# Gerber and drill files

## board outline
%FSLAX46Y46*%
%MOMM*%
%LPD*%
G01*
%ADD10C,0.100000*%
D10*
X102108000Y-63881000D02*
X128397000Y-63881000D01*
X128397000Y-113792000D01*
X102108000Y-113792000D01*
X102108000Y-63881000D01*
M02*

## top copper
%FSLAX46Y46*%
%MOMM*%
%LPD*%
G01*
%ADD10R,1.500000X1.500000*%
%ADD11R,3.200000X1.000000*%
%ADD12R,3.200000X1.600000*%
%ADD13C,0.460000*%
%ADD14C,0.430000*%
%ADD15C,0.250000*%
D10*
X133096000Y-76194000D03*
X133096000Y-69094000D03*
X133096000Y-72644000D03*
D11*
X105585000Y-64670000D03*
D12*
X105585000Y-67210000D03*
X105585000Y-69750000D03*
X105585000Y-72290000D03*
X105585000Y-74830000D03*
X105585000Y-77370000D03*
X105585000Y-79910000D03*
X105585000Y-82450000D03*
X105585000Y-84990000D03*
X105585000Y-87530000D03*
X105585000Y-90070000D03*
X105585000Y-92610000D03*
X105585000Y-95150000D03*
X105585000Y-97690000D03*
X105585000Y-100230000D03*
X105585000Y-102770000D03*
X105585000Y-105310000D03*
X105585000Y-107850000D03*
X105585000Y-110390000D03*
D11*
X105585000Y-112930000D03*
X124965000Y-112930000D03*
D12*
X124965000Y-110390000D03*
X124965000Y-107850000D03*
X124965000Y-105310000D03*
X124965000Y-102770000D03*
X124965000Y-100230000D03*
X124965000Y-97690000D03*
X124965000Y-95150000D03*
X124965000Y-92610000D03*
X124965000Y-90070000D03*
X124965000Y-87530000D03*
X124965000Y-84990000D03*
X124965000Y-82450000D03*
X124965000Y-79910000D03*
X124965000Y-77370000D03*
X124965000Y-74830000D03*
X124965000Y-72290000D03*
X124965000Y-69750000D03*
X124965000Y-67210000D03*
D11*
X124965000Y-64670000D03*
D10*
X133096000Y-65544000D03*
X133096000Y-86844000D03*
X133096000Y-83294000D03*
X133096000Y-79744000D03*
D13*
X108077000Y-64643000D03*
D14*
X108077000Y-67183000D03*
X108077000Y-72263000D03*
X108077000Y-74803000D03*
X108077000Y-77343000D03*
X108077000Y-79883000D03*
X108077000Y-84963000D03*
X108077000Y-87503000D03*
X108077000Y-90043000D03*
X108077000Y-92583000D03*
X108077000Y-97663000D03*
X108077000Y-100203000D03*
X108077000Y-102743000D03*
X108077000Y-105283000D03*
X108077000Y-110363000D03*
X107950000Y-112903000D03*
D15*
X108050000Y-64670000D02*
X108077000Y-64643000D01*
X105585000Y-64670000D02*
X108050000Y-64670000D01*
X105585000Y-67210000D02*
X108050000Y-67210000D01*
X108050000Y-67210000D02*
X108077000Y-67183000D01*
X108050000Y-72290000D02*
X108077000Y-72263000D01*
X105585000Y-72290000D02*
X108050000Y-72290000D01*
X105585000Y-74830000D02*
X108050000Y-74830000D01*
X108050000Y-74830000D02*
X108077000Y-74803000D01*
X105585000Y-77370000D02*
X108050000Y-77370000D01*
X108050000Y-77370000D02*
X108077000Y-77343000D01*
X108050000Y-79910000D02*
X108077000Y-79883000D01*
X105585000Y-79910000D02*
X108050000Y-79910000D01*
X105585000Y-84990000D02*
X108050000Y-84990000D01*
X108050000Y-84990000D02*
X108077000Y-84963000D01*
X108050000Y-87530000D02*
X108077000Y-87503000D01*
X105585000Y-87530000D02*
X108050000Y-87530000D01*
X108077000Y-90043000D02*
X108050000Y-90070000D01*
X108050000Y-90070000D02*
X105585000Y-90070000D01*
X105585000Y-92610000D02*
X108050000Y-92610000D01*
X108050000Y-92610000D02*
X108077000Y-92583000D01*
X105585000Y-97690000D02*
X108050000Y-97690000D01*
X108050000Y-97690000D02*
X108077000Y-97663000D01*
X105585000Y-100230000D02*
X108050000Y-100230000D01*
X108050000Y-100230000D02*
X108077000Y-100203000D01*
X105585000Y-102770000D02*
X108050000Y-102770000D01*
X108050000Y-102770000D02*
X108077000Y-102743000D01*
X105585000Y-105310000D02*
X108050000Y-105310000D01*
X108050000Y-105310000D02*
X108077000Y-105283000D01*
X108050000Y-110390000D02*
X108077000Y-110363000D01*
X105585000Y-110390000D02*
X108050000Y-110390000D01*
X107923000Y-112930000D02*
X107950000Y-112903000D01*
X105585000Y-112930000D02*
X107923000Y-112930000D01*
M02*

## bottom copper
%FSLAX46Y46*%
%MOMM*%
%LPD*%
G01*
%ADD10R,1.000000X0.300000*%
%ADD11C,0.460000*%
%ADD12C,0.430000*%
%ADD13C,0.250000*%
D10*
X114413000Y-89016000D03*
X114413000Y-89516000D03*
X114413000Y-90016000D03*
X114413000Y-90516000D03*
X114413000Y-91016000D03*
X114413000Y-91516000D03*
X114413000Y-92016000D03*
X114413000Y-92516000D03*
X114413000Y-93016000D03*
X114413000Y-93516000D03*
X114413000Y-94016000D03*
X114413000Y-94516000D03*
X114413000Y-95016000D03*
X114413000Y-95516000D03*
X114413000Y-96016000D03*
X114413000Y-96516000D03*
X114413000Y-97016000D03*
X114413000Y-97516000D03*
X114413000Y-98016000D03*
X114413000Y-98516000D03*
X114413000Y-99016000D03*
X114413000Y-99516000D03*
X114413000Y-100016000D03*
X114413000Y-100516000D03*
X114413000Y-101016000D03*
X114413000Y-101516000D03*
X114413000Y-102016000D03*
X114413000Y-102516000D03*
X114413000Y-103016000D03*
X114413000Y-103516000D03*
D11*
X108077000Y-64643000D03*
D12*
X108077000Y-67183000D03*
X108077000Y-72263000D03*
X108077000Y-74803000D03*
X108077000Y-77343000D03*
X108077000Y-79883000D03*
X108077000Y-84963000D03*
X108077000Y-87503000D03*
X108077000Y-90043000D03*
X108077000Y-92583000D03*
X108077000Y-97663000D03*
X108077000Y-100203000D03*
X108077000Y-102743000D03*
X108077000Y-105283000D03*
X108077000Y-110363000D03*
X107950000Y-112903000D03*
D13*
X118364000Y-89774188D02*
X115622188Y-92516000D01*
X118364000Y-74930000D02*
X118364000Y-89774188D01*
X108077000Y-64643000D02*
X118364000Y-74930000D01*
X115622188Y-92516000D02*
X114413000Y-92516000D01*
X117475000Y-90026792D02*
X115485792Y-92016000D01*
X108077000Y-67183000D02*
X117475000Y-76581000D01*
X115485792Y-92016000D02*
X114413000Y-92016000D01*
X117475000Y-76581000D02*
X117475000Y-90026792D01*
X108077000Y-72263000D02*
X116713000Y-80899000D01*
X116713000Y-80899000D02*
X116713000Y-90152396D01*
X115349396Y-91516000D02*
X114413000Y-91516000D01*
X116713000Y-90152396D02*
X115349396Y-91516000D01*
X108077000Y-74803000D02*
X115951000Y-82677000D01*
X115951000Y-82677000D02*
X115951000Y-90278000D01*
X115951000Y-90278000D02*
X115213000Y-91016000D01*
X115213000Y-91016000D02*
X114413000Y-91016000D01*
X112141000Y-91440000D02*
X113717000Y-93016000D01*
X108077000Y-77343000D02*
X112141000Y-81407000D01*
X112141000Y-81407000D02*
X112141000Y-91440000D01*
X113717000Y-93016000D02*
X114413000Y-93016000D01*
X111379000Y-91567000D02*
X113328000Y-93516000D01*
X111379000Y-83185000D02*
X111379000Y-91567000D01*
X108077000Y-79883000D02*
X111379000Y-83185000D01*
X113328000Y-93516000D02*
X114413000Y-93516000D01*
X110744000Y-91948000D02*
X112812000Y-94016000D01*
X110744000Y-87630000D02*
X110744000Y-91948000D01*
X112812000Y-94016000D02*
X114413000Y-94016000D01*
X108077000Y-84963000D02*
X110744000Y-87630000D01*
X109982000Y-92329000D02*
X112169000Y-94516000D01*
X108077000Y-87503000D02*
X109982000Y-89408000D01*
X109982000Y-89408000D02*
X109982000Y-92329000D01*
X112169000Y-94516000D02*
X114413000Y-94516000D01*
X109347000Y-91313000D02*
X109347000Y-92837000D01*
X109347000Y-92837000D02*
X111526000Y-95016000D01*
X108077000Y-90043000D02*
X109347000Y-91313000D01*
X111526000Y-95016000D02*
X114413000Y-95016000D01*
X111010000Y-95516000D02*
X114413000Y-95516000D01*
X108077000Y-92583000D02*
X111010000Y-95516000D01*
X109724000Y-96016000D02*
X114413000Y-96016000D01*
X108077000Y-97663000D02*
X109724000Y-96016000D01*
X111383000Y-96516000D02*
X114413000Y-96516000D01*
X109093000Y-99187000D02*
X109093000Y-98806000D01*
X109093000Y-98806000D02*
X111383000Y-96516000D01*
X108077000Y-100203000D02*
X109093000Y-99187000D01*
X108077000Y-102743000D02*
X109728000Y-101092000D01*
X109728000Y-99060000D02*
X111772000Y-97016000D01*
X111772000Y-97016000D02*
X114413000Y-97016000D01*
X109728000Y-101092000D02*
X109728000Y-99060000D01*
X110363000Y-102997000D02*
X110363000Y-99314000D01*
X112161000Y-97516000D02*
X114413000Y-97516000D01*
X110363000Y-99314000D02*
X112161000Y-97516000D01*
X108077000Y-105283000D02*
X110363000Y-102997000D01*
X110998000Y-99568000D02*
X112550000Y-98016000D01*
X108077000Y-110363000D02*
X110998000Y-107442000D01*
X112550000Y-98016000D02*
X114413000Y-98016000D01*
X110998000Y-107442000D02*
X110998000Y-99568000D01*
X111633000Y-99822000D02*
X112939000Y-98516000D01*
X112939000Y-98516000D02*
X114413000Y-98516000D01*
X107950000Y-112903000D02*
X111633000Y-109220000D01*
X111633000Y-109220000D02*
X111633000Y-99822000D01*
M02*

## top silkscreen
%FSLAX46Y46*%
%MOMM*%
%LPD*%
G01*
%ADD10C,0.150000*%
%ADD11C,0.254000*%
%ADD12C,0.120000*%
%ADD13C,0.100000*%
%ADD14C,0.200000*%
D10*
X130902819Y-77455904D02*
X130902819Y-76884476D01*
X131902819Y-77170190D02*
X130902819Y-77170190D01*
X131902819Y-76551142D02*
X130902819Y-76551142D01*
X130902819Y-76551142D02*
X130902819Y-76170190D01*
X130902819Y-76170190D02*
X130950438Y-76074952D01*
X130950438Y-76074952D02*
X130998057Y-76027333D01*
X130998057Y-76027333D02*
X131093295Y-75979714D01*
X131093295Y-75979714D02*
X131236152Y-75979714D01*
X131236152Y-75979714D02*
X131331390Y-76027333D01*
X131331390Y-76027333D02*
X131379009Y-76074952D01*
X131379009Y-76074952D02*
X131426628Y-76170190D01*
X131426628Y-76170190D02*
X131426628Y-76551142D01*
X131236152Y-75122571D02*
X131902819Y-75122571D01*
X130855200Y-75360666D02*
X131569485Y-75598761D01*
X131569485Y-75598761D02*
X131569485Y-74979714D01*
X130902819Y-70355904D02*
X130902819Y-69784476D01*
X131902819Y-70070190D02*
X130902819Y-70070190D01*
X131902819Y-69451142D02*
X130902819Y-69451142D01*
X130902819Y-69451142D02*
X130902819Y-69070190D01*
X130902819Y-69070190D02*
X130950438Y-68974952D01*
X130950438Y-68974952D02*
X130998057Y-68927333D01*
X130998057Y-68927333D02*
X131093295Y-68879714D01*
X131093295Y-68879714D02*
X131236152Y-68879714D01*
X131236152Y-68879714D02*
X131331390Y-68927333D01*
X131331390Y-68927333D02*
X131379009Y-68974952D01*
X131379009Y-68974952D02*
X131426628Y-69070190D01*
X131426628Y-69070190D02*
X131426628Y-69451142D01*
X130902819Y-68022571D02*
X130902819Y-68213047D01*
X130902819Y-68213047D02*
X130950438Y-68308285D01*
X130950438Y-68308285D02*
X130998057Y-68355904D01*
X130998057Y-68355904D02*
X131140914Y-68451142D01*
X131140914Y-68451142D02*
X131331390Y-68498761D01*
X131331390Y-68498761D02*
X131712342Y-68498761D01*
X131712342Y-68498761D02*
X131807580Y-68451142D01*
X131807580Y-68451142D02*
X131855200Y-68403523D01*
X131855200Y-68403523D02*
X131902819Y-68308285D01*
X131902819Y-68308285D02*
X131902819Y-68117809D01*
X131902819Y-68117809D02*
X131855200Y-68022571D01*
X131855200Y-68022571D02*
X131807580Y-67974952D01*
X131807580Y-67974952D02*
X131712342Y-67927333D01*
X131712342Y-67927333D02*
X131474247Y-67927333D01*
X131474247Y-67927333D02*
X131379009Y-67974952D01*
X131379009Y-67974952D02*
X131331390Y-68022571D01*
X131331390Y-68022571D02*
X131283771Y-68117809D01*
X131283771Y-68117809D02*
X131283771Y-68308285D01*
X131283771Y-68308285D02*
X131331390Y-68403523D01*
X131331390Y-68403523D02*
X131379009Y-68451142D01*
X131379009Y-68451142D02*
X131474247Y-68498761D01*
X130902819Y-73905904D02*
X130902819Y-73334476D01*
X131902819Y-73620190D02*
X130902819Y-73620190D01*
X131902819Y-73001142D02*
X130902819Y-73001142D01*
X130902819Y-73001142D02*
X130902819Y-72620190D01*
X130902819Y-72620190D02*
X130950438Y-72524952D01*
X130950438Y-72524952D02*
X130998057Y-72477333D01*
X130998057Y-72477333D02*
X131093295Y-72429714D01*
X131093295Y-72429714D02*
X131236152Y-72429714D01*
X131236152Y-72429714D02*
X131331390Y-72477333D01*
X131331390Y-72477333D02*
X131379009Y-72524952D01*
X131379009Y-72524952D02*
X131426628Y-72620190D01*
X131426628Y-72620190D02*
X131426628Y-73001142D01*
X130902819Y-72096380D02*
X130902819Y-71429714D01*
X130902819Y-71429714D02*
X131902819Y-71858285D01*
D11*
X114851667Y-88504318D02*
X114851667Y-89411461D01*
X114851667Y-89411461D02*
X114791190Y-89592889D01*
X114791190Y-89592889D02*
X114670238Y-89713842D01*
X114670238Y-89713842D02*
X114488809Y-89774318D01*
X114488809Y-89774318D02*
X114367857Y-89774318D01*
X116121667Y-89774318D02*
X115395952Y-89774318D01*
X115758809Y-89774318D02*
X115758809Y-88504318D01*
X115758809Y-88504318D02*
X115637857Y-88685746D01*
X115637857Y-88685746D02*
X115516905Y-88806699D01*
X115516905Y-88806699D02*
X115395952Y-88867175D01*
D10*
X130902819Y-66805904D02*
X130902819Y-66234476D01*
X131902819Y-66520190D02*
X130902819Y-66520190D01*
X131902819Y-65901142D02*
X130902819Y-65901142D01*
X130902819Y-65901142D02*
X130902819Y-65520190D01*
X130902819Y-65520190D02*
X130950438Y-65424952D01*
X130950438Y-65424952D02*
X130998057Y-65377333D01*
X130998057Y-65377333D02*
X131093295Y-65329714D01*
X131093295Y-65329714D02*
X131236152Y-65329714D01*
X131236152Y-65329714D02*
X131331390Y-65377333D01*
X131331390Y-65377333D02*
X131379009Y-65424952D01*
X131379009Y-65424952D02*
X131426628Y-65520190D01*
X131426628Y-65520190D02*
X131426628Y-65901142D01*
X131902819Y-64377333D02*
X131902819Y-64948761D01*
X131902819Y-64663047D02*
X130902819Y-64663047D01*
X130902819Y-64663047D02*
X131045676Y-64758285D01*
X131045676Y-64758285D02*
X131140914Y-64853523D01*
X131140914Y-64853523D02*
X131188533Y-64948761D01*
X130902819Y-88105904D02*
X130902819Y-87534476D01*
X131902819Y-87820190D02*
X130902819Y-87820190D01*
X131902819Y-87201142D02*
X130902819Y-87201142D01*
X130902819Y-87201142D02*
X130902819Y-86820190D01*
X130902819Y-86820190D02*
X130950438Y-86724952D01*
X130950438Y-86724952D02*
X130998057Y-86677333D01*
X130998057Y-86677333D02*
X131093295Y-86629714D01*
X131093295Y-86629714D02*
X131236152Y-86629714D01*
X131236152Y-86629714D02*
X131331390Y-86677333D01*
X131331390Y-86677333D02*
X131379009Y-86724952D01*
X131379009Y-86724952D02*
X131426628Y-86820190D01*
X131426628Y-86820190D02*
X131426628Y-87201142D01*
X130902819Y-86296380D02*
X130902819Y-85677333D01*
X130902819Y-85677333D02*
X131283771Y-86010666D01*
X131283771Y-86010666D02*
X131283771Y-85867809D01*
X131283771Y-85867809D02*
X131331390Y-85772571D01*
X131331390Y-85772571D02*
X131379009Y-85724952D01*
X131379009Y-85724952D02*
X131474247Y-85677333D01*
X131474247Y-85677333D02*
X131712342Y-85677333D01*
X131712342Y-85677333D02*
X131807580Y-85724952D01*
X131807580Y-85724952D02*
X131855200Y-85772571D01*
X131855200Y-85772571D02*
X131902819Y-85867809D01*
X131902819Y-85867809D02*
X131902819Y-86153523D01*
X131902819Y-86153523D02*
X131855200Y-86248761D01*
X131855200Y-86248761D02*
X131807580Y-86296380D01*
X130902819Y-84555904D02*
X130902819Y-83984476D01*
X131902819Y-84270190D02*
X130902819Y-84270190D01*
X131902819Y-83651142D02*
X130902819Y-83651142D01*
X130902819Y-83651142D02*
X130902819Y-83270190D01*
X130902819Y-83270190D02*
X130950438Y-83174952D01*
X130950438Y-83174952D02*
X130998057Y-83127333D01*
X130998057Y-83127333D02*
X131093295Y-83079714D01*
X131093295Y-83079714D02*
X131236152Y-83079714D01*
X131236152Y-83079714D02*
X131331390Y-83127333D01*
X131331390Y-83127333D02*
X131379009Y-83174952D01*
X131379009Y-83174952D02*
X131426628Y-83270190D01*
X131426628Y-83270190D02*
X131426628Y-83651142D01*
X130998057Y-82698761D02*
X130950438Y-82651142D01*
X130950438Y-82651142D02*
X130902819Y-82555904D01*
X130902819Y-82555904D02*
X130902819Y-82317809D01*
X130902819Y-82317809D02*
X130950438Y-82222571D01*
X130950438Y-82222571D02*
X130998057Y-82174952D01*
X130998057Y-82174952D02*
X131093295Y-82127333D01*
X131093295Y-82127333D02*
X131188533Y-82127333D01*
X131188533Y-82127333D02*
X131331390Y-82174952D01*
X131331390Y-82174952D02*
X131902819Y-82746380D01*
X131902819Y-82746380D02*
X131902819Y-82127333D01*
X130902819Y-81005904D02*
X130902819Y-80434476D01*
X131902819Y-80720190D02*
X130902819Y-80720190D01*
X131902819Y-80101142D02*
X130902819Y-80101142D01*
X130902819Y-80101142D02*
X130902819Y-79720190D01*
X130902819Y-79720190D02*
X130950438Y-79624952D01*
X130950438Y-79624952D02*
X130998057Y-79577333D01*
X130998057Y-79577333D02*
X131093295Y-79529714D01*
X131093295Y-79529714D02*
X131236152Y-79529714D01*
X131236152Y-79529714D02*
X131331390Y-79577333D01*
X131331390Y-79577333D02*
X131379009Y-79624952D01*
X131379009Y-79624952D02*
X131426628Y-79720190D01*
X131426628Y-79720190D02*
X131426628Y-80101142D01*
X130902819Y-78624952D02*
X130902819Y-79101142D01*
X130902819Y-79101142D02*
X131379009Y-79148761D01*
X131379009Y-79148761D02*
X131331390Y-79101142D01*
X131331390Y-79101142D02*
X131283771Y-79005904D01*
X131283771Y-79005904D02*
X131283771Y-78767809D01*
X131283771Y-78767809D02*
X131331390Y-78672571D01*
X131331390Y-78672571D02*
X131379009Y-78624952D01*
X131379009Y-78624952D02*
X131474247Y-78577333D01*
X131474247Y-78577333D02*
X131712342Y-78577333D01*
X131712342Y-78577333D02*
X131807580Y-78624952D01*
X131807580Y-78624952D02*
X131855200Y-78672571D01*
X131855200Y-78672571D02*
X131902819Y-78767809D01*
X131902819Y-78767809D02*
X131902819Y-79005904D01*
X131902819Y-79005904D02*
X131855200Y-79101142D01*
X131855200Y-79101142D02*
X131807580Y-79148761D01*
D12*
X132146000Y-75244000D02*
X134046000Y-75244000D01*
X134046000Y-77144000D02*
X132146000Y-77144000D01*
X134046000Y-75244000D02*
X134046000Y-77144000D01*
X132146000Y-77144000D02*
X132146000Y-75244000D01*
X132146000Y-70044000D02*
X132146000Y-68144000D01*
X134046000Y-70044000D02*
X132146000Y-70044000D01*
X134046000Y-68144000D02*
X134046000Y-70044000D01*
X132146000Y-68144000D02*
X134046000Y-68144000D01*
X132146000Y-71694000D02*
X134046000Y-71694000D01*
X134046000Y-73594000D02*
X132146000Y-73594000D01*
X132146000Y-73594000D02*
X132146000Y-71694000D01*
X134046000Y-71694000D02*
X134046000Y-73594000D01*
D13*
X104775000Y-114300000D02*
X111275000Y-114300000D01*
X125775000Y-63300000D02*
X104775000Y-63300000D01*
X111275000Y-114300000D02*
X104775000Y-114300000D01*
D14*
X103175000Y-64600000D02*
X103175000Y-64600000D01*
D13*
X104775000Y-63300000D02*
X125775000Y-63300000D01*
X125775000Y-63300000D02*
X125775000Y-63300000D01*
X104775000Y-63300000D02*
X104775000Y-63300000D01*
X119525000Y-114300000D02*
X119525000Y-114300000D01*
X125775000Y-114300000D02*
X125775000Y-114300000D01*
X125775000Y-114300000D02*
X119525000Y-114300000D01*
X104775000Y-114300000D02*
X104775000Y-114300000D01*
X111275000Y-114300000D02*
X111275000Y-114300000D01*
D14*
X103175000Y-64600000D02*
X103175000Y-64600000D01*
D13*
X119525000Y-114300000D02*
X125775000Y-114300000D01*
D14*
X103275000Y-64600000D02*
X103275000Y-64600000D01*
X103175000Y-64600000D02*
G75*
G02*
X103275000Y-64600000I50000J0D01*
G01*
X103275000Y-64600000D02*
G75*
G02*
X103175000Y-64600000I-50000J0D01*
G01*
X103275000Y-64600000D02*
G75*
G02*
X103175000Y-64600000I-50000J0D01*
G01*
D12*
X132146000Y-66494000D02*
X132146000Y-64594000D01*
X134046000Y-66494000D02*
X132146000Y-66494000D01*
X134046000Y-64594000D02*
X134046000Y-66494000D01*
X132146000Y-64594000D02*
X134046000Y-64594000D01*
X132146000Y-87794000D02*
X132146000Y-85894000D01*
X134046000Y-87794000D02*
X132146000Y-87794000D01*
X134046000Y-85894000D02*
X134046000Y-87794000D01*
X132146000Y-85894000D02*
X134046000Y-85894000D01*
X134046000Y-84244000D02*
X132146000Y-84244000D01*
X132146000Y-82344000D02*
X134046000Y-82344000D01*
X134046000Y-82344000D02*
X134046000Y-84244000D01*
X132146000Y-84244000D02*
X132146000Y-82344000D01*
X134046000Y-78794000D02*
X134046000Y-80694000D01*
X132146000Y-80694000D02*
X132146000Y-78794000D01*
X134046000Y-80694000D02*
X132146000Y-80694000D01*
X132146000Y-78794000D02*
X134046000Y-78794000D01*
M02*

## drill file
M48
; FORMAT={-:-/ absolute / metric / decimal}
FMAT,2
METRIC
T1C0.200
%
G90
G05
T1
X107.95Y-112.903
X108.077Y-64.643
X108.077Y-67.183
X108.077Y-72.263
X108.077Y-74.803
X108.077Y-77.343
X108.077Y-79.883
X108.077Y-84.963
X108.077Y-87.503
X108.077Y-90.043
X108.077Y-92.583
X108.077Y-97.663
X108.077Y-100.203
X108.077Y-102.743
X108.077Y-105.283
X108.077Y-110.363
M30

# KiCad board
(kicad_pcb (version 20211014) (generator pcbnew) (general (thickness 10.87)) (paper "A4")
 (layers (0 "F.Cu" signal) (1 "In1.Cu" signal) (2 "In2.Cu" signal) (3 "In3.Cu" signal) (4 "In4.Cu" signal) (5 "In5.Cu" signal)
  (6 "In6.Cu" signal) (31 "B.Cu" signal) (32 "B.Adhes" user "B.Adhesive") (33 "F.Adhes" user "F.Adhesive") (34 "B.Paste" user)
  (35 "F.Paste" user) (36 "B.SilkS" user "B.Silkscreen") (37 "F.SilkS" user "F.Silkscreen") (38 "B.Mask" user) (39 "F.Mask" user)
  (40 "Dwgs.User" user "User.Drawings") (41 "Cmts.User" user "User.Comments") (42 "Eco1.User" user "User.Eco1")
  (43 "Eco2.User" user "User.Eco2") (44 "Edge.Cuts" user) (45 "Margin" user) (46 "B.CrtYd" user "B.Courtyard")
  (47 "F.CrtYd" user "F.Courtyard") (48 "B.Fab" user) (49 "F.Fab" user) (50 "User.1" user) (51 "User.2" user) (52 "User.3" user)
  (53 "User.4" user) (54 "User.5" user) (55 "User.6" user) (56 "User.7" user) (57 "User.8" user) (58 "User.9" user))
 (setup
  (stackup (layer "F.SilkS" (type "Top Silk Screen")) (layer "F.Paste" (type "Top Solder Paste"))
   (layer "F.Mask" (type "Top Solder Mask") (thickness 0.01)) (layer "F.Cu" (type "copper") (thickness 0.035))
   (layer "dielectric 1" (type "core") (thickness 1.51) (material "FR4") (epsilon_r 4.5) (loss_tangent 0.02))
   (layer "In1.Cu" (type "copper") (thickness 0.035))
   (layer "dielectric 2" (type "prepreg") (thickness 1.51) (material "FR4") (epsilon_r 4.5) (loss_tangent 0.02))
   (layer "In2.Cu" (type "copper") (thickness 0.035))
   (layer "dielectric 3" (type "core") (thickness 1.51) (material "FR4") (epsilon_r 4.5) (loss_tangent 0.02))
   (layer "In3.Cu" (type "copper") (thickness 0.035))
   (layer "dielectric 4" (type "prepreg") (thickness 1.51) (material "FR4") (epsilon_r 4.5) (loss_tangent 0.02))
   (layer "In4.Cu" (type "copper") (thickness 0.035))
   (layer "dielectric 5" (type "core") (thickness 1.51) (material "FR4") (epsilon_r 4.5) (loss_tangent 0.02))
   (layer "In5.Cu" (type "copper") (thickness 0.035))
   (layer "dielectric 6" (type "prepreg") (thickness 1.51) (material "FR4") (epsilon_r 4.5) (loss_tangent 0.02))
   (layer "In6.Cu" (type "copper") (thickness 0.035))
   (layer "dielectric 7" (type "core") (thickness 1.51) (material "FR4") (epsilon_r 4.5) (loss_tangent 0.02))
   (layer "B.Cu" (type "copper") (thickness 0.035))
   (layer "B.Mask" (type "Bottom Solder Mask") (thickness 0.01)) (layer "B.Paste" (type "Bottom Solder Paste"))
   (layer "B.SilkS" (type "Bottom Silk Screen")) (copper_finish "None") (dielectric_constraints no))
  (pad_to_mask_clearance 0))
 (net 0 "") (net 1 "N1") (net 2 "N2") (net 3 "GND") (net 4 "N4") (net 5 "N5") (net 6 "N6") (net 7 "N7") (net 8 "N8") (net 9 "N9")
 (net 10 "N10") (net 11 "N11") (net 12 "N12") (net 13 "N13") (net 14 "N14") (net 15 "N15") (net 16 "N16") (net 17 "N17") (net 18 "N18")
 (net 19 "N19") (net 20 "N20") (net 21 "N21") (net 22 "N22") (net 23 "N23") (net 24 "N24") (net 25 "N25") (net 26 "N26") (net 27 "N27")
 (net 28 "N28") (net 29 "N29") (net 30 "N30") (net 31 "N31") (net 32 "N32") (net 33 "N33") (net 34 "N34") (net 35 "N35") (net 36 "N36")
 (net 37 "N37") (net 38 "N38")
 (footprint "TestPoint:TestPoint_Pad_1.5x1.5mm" (layer "F.Cu") (at 133.096 76.194 90)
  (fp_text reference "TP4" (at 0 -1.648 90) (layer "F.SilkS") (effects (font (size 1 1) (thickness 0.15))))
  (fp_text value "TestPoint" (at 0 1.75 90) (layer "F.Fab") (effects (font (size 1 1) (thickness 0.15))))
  (fp_line (start 0.95 -0.95) (end 0.95 0.95) (layer "F.SilkS") (width 0.12))
  (fp_line (start -0.95 0.95) (end -0.95 -0.95) (layer "F.SilkS") (width 0.12))
  (fp_line (start 0.95 0.95) (end -0.95 0.95) (layer "F.SilkS") (width 0.12))
  (fp_line (start -0.95 -0.95) (end 0.95 -0.95) (layer "F.SilkS") (width 0.12))
  (pad "1" smd rect (at 0 0 90) (size 1.5 1.5) (layers "F.Cu" "F.Mask") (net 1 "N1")))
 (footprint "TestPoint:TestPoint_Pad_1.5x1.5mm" (layer "F.Cu") (at 133.096 69.094 90)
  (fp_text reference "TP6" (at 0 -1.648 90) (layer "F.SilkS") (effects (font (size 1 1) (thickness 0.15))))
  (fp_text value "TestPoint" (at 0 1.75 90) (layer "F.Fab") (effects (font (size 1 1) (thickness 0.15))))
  (fp_line (start -0.95 -0.95) (end 0.95 -0.95) (layer "F.SilkS") (width 0.12))
  (fp_line (start -0.95 0.95) (end -0.95 -0.95) (layer "F.SilkS") (width 0.12))
  (fp_line (start 0.95 0.95) (end -0.95 0.95) (layer "F.SilkS") (width 0.12))
  (fp_line (start 0.95 -0.95) (end 0.95 0.95) (layer "F.SilkS") (width 0.12))
  (pad "1" smd rect (at 0 0 90) (size 1.5 1.5) (layers "F.Cu" "F.Mask") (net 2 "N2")))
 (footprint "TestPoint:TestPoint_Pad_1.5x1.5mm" (layer "F.Cu") (at 133.096 72.644 90)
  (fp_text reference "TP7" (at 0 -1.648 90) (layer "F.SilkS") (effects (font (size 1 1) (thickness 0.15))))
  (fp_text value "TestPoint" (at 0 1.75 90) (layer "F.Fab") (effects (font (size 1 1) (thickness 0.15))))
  (fp_line (start 0.95 -0.95) (end 0.95 0.95) (layer "F.SilkS") (width 0.12))
  (fp_line (start -0.95 0.95) (end -0.95 -0.95) (layer "F.SilkS") (width 0.12))
  (fp_line (start -0.95 -0.95) (end 0.95 -0.95) (layer "F.SilkS") (width 0.12))
  (fp_line (start 0.95 0.95) (end -0.95 0.95) (layer "F.SilkS") (width 0.12))
  (pad "1" smd rect (at 0 0 90) (size 1.5 1.5) (layers "F.Cu" "F.Mask") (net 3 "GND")))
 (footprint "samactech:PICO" (layer "F.Cu") (at 104.775 114.3)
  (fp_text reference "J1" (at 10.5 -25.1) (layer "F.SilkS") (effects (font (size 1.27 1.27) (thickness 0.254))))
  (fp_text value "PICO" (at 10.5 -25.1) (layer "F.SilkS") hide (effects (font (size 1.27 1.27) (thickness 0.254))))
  (fp_line (start 0 0) (end 6.5 0) (layer "F.SilkS") (width 0.1))
  (fp_line (start 21 -51) (end 0 -51) (layer "F.SilkS") (width 0.1))
  (fp_line (start 6.5 0) (end 0 0) (layer "F.SilkS") (width 0.1))
  (fp_line (start -1.6 -49.7) (end -1.6 -49.7) (layer "F.SilkS") (width 0.2))
  (fp_line (start 0 -51) (end 21 -51) (layer "F.SilkS") (width 0.1))
  (fp_line (start 21 -51) (end 21 -51) (layer "F.SilkS") (width 0.1))
  (fp_line (start 0 -51) (end 0 -51) (layer "F.SilkS") (width 0.1))
  (fp_line (start 14.75 0) (end 14.75 0) (layer "F.SilkS") (width 0.1))
  (fp_line (start 21 0) (end 21 0) (layer "F.SilkS") (width 0.1))
  (fp_line (start 21 0) (end 14.75 0) (layer "F.SilkS") (width 0.1))
  (fp_line (start 0 0) (end 0 0) (layer "F.SilkS") (width 0.1))
  (fp_line (start 6.5 0) (end 6.5 0) (layer "F.SilkS") (width 0.1))
  (fp_line (start -1.6 -49.7) (end -1.6 -49.7) (layer "F.SilkS") (width 0.2))
  (fp_line (start 14.75 0) (end 21 0) (layer "F.SilkS") (width 0.1))
  (fp_line (start -1.5 -49.7) (end -1.5 -49.7) (layer "F.SilkS") (width 0.2))
  (fp_arc (start -1.6 -49.7) (mid -1.55 -49.75) (end -1.5 -49.7) (layer "F.SilkS") (width 0.2))
  (fp_arc (start -1.5 -49.7) (mid -1.55 -49.65) (end -1.6 -49.7) (layer "F.SilkS") (width 0.2))
  (fp_arc (start -1.5 -49.7) (mid -1.55 -49.65) (end -1.6 -49.7) (layer "F.SilkS") (width 0.2))
  (pad "1" smd rect (at 0.81 -49.63 90) (size 1 3.2) (layers "F.Cu" "F.Paste" "F.Mask") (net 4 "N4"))
  (pad "2" smd rect (at 0.81 -47.09 90) (size 1.6 3.2) (layers "F.Cu" "F.Paste" "F.Mask") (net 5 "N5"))
  (pad "3" smd rect (at 0.81 -44.55 90) (size 1.6 3.2) (layers "F.Cu" "F.Paste" "F.Mask") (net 3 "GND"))
  (pad "4" smd rect (at 0.81 -42.01 90) (size 1.6 3.2) (layers "F.Cu" "F.Paste" "F.Mask") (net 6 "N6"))
  (pad "5" smd rect (at 0.81 -39.47 90) (size 1.6 3.2) (layers "F.Cu" "F.Paste" "F.Mask") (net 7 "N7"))
  (pad "6" smd rect (at 0.81 -36.93 90) (size 1.6 3.2) (layers "F.Cu" "F.Paste" "F.Mask") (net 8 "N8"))
  (pad "7" smd rect (at 0.81 -34.39 90) (size 1.6 3.2) (layers "F.Cu" "F.Paste" "F.Mask") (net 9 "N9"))
  (pad "8" smd rect (at 0.81 -31.85 90) (size 1.6 3.2) (layers "F.Cu" "F.Paste" "F.Mask") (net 3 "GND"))
  (pad "9" smd rect (at 0.81 -29.31 90) (size 1.6 3.2) (layers "F.Cu" "F.Paste" "F.Mask") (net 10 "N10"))
  (pad "10" smd rect (at 0.81 -26.77 90) (size 1.6 3.2) (layers "F.Cu" "F.Paste" "F.Mask") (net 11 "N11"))
  (pad "11" smd rect (at 0.81 -24.23 90) (size 1.6 3.2) (layers "F.Cu" "F.Paste" "F.Mask") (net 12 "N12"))
  (pad "12" smd rect (at 0.81 -21.69 90) (size 1.6 3.2) (layers "F.Cu" "F.Paste" "F.Mask") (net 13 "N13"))
  (pad "13" smd rect (at 0.81 -19.15 90) (size 1.6 3.2) (layers "F.Cu" "F.Paste" "F.Mask") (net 3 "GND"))
  (pad "14" smd rect (at 0.81 -16.61 90) (size 1.6 3.2) (layers "F.Cu" "F.Paste" "F.Mask") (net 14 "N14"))
  (pad "15" smd rect (at 0.81 -14.07 90) (size 1.6 3.2) (layers "F.Cu" "F.Paste" "F.Mask") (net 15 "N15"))
  (pad "16" smd rect (at 0.81 -11.53 90) (size 1.6 3.2) (layers "F.Cu" "F.Paste" "F.Mask") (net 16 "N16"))
  (pad "17" smd rect (at 0.81 -8.99 90) (size 1.6 3.2) (layers "F.Cu" "F.Paste" "F.Mask") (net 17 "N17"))
  (pad "18" smd rect (at 0.81 -6.45 90) (size 1.6 3.2) (layers "F.Cu" "F.Paste" "F.Mask") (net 3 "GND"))
  (pad "19" smd rect (at 0.81 -3.91 90) (size 1.6 3.2) (layers "F.Cu" "F.Paste" "F.Mask") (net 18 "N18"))
  (pad "20" smd rect (at 0.81 -1.37 90) (size 1 3.2) (layers "F.Cu" "F.Paste" "F.Mask") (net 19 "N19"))
  (pad "21" smd rect (at 20.19 -1.37 90) (size 1 3.2) (layers "F.Cu" "F.Paste" "F.Mask") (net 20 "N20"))
  (pad "22" smd rect (at 20.19 -3.91 90) (size 1.6 3.2) (layers "F.Cu" "F.Paste" "F.Mask") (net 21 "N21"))
  (pad "23" smd rect (at 20.19 -6.45 90) (size 1.6 3.2) (layers "F.Cu" "F.Paste" "F.Mask") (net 3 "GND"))
  (pad "24" smd rect (at 20.19 -8.99 90) (size 1.6 3.2) (layers "F.Cu" "F.Paste" "F.Mask") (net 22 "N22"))
  (pad "25" smd rect (at 20.19 -11.53 90) (size 1.6 3.2) (layers "F.Cu" "F.Paste" "F.Mask") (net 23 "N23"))
  (pad "26" smd rect (at 20.19 -14.07 90) (size 1.6 3.2) (layers "F.Cu" "F.Paste" "F.Mask") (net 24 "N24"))
  (pad "27" smd rect (at 20.19 -16.61 90) (size 1.6 3.2) (layers "F.Cu" "F.Paste" "F.Mask") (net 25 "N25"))
  (pad "28" smd rect (at 20.19 -19.15 90) (size 1.6 3.2) (layers "F.Cu" "F.Paste" "F.Mask") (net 3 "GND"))
  (pad "29" smd rect (at 20.19 -21.69 90) (size 1.6 3.2) (layers "F.Cu" "F.Paste" "F.Mask") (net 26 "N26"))
  (pad "30" smd rect (at 20.19 -24.23 90) (size 1.6 3.2) (layers "F.Cu" "F.Paste" "F.Mask") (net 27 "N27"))
  (pad "31" smd rect (at 20.19 -26.77 90) (size 1.6 3.2) (layers "F.Cu" "F.Paste" "F.Mask") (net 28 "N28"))
  (pad "32" smd rect (at 20.19 -29.31 90) (size 1.6 3.2) (layers "F.Cu" "F.Paste" "F.Mask") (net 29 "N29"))
  (pad "33" smd rect (at 20.19 -31.85 90) (size 1.6 3.2) (layers "F.Cu" "F.Paste" "F.Mask") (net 3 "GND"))
  (pad "34" smd rect (at 20.19 -34.39 90) (size 1.6 3.2) (layers "F.Cu" "F.Paste" "F.Mask") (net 2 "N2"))
  (pad "35" smd rect (at 20.19 -36.93 90) (size 1.6 3.2) (layers "F.Cu" "F.Paste" "F.Mask") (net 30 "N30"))
  (pad "36" smd rect (at 20.19 -39.47 90) (size 1.6 3.2) (layers "F.Cu" "F.Paste" "F.Mask") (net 1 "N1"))
  (pad "37" smd rect (at 20.19 -42.01 90) (size 1.6 3.2) (layers "F.Cu" "F.Paste" "F.Mask") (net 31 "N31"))
  (pad "38" smd rect (at 20.19 -44.55 90) (size 1.6 3.2) (layers "F.Cu" "F.Paste" "F.Mask") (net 3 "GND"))
  (pad "39" smd rect (at 20.19 -47.09 90) (size 1.6 3.2) (layers "F.Cu" "F.Paste" "F.Mask") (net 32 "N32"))
  (pad "40" smd rect (at 20.19 -49.63 90) (size 1 3.2) (layers "F.Cu" "F.Paste" "F.Mask") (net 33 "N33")))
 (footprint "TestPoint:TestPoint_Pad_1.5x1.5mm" (layer "F.Cu") (at 133.096 65.544 90)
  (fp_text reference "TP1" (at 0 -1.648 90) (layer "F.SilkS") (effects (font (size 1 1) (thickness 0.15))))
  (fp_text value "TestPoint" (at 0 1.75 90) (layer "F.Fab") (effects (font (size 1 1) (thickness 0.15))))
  (fp_line (start -0.95 -0.95) (end 0.95 -0.95) (layer "F.SilkS") (width 0.12))
  (fp_line (start -0.95 0.95) (end -0.95 -0.95) (layer "F.SilkS") (width 0.12))
  (fp_line (start 0.95 0.95) (end -0.95 0.95) (layer "F.SilkS") (width 0.12))
  (fp_line (start 0.95 -0.95) (end 0.95 0.95) (layer "F.SilkS") (width 0.12))
  (pad "1" smd rect (at 0 0 90) (size 1.5 1.5) (layers "F.Cu" "F.Mask") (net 33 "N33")))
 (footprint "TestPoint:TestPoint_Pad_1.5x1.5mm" (layer "F.Cu") (at 133.096 86.844 90)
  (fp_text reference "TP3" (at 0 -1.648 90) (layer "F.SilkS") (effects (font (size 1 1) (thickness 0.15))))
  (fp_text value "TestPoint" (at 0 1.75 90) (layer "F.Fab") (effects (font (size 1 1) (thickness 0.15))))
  (fp_line (start -0.95 -0.95) (end 0.95 -0.95) (layer "F.SilkS") (width 0.12))
  (fp_line (start -0.95 0.95) (end -0.95 -0.95) (layer "F.SilkS") (width 0.12))
  (fp_line (start 0.95 0.95) (end -0.95 0.95) (layer "F.SilkS") (width 0.12))
  (fp_line (start 0.95 -0.95) (end 0.95 0.95) (layer "F.SilkS") (width 0.12))
  (pad "1" smd rect (at 0 0 90) (size 1.5 1.5) (layers "F.Cu" "F.Mask") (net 31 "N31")))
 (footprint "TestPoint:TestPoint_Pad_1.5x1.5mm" (layer "F.Cu") (at 133.096 83.294 90)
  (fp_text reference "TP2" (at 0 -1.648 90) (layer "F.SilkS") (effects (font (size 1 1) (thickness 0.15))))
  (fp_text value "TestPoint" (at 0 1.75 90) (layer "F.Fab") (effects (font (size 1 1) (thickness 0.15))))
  (fp_line (start -0.95 0.95) (end -0.95 -0.95) (layer "F.SilkS") (width 0.12))
  (fp_line (start 0.95 -0.95) (end 0.95 0.95) (layer "F.SilkS") (width 0.12))
  (fp_line (start 0.95 0.95) (end -0.95 0.95) (layer "F.SilkS") (width 0.12))
  (fp_line (start -0.95 -0.95) (end 0.95 -0.95) (layer "F.SilkS") (width 0.12))
  (pad "1" smd rect (at 0 0 90) (size 1.5 1.5) (layers "F.Cu" "F.Mask") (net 32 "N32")))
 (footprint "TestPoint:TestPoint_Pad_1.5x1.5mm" (layer "F.Cu") (at 133.096 79.744 90)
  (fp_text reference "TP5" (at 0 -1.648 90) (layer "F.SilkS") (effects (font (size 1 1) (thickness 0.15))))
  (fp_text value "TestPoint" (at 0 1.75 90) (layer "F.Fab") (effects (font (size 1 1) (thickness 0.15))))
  (fp_line (start 0.95 0.95) (end -0.95 0.95) (layer "F.SilkS") (width 0.12))
  (fp_line (start -0.95 -0.95) (end 0.95 -0.95) (layer "F.SilkS") (width 0.12))
  (fp_line (start -0.95 0.95) (end -0.95 -0.95) (layer "F.SilkS") (width 0.12))
  (fp_line (start 0.95 -0.95) (end 0.95 0.95) (layer "F.SilkS") (width 0.12))
  (pad "1" smd rect (at 0 0 90) (size 1.5 1.5) (layers "F.Cu" "F.Mask") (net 30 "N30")))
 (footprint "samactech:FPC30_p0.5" (layer "B.Cu") (at 116.913 96.266 -90)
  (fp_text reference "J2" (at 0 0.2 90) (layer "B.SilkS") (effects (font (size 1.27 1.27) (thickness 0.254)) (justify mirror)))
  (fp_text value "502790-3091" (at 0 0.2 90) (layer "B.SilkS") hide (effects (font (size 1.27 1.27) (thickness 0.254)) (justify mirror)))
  (pad "1" smd rect (at -7.25 2.5 270) (size 0.3 1) (layers "B.Cu" "B.Paste" "B.Mask") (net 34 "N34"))
  (pad "2" smd rect (at -6.75 2.5 270) (size 0.3 1) (layers "B.Cu" "B.Paste" "B.Mask") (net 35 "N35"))
  (pad "3" smd rect (at -6.25 2.5 270) (size 0.3 1) (layers "B.Cu" "B.Paste" "B.Mask") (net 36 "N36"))
  (pad "4" smd rect (at -5.75 2.5 270) (size 0.3 1) (layers "B.Cu" "B.Paste" "B.Mask") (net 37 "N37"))
  (pad "5" smd rect (at -5.25 2.5 270) (size 0.3 1) (layers "B.Cu" "B.Paste" "B.Mask") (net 7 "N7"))
  (pad "6" smd rect (at -4.75 2.5 270) (size 0.3 1) (layers "B.Cu" "B.Paste" "B.Mask") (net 6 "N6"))
  (pad "7" smd rect (at -4.25 2.5 270) (size 0.3 1) (layers "B.Cu" "B.Paste" "B.Mask") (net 5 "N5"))
  (pad "8" smd rect (at -3.75 2.5 270) (size 0.3 1) (layers "B.Cu" "B.Paste" "B.Mask") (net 4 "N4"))
  (pad "9" smd rect (at -3.25 2.5 270) (size 0.3 1) (layers "B.Cu" "B.Paste" "B.Mask") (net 8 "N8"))
  (pad "10" smd rect (at -2.75 2.5 270) (size 0.3 1) (layers "B.Cu" "B.Paste" "B.Mask") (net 9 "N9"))
  (pad "11" smd rect (at -2.25 2.5 270) (size 0.3 1) (layers "B.Cu" "B.Paste" "B.Mask") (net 10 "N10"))
  (pad "12" smd rect (at -1.75 2.5 270) (size 0.3 1) (layers "B.Cu" "B.Paste" "B.Mask") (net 11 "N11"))
  (pad "13" smd rect (at -1.25 2.5 270) (size 0.3 1) (layers "B.Cu" "B.Paste" "B.Mask") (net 12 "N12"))
  (pad "14" smd rect (at -0.75 2.5 270) (size 0.3 1) (layers "B.Cu" "B.Paste" "B.Mask") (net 13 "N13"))
  (pad "15" smd rect (at -0.25 2.5 270) (size 0.3 1) (layers "B.Cu" "B.Paste" "B.Mask") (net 14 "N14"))
  (pad "16" smd rect (at 0.25 2.5 270) (size 0.3 1) (layers "B.Cu" "B.Paste" "B.Mask") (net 15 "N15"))
  (pad "17" smd rect (at 0.75 2.5 270) (size 0.3 1) (layers "B.Cu" "B.Paste" "B.Mask") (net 16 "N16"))
  (pad "18" smd rect (at 1.25 2.5 270) (size 0.3 1) (layers "B.Cu" "B.Paste" "B.Mask") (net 17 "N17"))
  (pad "19" smd rect (at 1.75 2.5 270) (size 0.3 1) (layers "B.Cu" "B.Paste" "B.Mask") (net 18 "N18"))
  (pad "20" smd rect (at 2.25 2.5 270) (size 0.3 1) (layers "B.Cu" "B.Paste" "B.Mask") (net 19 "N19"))
  (pad "21" smd rect (at 2.75 2.5 270) (size 0.3 1) (layers "B.Cu" "B.Paste" "B.Mask") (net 29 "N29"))
  (pad "22" smd rect (at 3.25 2.5 270) (size 0.3 1) (layers "B.Cu" "B.Paste" "B.Mask") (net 28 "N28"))
  (pad "23" smd rect (at 3.75 2.5 270) (size 0.3 1) (layers "B.Cu" "B.Paste" "B.Mask") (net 26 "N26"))
  (pad "24" smd rect (at 4.25 2.5 270) (size 0.3 1) (layers "B.Cu" "B.Paste" "B.Mask") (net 25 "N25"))
  (pad "25" smd rect (at 4.75 2.5 270) (size 0.3 1) (layers "B.Cu" "B.Paste" "B.Mask") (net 24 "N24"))
  (pad "26" smd rect (at 5.25 2.5 270) (size 0.3 1) (layers "B.Cu" "B.Paste" "B.Mask") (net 23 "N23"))
  (pad "27" smd rect (at 5.75 2.5 270) (size 0.3 1) (layers "B.Cu" "B.Paste" "B.Mask") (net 22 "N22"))
  (pad "28" smd rect (at 6.25 2.5 270) (size 0.3 1) (layers "B.Cu" "B.Paste" "B.Mask") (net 21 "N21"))
  (pad "29" smd rect (at 6.75 2.5 270) (size 0.3 1) (layers "B.Cu" "B.Paste" "B.Mask") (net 20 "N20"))
  (pad "30" smd rect (at 7.25 2.5 270) (size 0.3 1) (layers "B.Cu" "B.Paste" "B.Mask") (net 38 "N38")))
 (gr_rect (start 102.108 63.881) (end 128.397 113.792) (layer "Edge.Cuts") (width 0.1) (fill none))
 (segment (start 108.05 64.67) (end 108.077 64.643) (width 0.25) (layer "F.Cu") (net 4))
 (segment (start 105.585 64.67) (end 108.05 64.67) (width 0.25) (layer "F.Cu") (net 4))
 (via (at 108.077 64.643) (size 0.46) (drill 0.2) (layers "F.Cu" "B.Cu") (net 4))
 (segment (start 118.364 89.774188) (end 115.622188 92.516) (width 0.25) (layer "B.Cu") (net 4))
 (segment (start 118.364 74.93) (end 118.364 89.774188) (width 0.25) (layer "B.Cu") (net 4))
 (segment (start 108.077 64.643) (end 118.364 74.93) (width 0.25) (layer "B.Cu") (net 4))
 (segment (start 115.622188 92.516) (end 114.413 92.516) (width 0.25) (layer "B.Cu") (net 4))
 (segment (start 105.585 67.21) (end 108.05 67.21) (width 0.25) (layer "F.Cu") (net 5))
 (segment (start 108.05 67.21) (end 108.077 67.183) (width 0.25) (layer "F.Cu") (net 5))
 (via (at 108.077 67.183) (size 0.43) (drill 0.2) (layers "F.Cu" "B.Cu") (free) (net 5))
 (segment (start 117.475 90.026792) (end 115.485792 92.016) (width 0.25) (layer "B.Cu") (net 5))
 (segment (start 108.077 67.183) (end 117.475 76.581) (width 0.25) (layer "B.Cu") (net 5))
 (segment (start 115.485792 92.016) (end 114.413 92.016) (width 0.25) (layer "B.Cu") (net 5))
 (segment (start 117.475 76.581) (end 117.475 90.026792) (width 0.25) (layer "B.Cu") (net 5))
 (segment (start 108.05 72.29) (end 108.077 72.263) (width 0.25) (layer "F.Cu") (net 6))
 (segment (start 105.585 72.29) (end 108.05 72.29) (width 0.25) (layer "F.Cu") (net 6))
 (via (at 108.077 72.263) (size 0.43) (drill 0.2) (layers "F.Cu" "B.Cu") (free) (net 6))
 (segment (start 108.077 72.263) (end 116.713 80.899) (width 0.25) (layer "B.Cu") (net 6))
 (segment (start 116.713 80.899) (end 116.713 90.152396) (width 0.25) (layer "B.Cu") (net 6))
 (segment (start 115.349396 91.516) (end 114.413 91.516) (width 0.25) (layer "B.Cu") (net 6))
 (segment (start 116.713 90.152396) (end 115.349396 91.516) (width 0.25) (layer "B.Cu") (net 6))
 (segment (start 105.585 74.83) (end 108.05 74.83) (width 0.25) (layer "F.Cu") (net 7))
 (segment (start 108.05 74.83) (end 108.077 74.803) (width 0.25) (layer "F.Cu") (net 7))
 (via (at 108.077 74.803) (size 0.43) (drill 0.2) (layers "F.Cu" "B.Cu") (free) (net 7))
 (segment (start 108.077 74.803) (end 115.951 82.677) (width 0.25) (layer "B.Cu") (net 7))
 (segment (start 115.951 82.677) (end 115.951 90.278) (width 0.25) (layer "B.Cu") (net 7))
 (segment (start 115.951 90.278) (end 115.213 91.016) (width 0.25) (layer "B.Cu") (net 7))
 (segment (start 115.213 91.016) (end 114.413 91.016) (width 0.25) (layer "B.Cu") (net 7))
 (segment (start 105.585 77.37) (end 108.05 77.37) (width 0.25) (layer "F.Cu") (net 8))
 (segment (start 108.05 77.37) (end 108.077 77.343) (width 0.25) (layer "F.Cu") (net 8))
 (via (at 108.077 77.343) (size 0.43) (drill 0.2) (layers "F.Cu" "B.Cu") (free) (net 8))
 (segment (start 112.141 91.44) (end 113.717 93.016) (width 0.25) (layer "B.Cu") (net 8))
 (segment (start 108.077 77.343) (end 112.141 81.407) (width 0.25) (layer "B.Cu") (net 8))
 (segment (start 112.141 81.407) (end 112.141 91.44) (width 0.25) (layer "B.Cu") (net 8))
 (segment (start 113.717 93.016) (end 114.413 93.016) (width 0.25) (layer "B.Cu") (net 8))
 (segment (start 108.05 79.91) (end 108.077 79.883) (width 0.25) (layer "F.Cu") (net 9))
 (segment (start 105.585 79.91) (end 108.05 79.91) (width 0.25) (layer "F.Cu") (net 9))
 (via (at 108.077 79.883) (size 0.43) (drill 0.2) (layers "F.Cu" "B.Cu") (free) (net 9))
 (segment (start 111.379 91.567) (end 113.328 93.516) (width 0.25) (layer "B.Cu") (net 9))
 (segment (start 111.379 83.185) (end 111.379 91.567) (width 0.25) (layer "B.Cu") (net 9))
 (segment (start 108.077 79.883) (end 111.379 83.185) (width 0.25) (layer "B.Cu") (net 9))
 (segment (start 113.328 93.516) (end 114.413 93.516) (width 0.25) (layer "B.Cu") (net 9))
 (segment (start 105.585 84.99) (end 108.05 84.99) (width 0.25) (layer "F.Cu") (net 10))
 (segment (start 108.05 84.99) (end 108.077 84.963) (width 0.25) (layer "F.Cu") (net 10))
 (via (at 108.077 84.963) (size 0.43) (drill 0.2) (layers "F.Cu" "B.Cu") (free) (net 10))
 (segment (start 110.744 91.948) (end 112.812 94.016) (width 0.25) (layer "B.Cu") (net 10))
 (segment (start 110.744 87.63) (end 110.744 91.948) (width 0.25) (layer "B.Cu") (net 10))
 (segment (start 112.812 94.016) (end 114.413 94.016) (width 0.25) (layer "B.Cu") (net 10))
 (segment (start 108.077 84.963) (end 110.744 87.63) (width 0.25) (layer "B.Cu") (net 10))
 (segment (start 108.05 87.53) (end 108.077 87.503) (width 0.25) (layer "F.Cu") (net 11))
 (segment (start 105.585 87.53) (end 108.05 87.53) (width 0.25) (layer "F.Cu") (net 11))
 (via (at 108.077 87.503) (size 0.43) (drill 0.2) (layers "F.Cu" "B.Cu") (free) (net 11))
 (segment (start 109.982 92.329) (end 112.169 94.516) (width 0.25) (layer "B.Cu") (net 11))
 (segment (start 108.077 87.503) (end 109.982 89.408) (width 0.25) (layer "B.Cu") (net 11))
 (segment (start 109.982 89.408) (end 109.982 92.329) (width 0.25) (layer "B.Cu") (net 11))
 (segment (start 112.169 94.516) (end 114.413 94.516) (width 0.25) (layer "B.Cu") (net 11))
 (segment (start 108.077 90.043) (end 108.05 90.07) (width 0.25) (layer "F.Cu") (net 12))
 (segment (start 108.05 90.07) (end 105.585 90.07) (width 0.25) (layer "F.Cu") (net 12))
 (via (at 108.077 90.043) (size 0.43) (drill 0.2) (layers "F.Cu" "B.Cu") (free) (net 12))
 (segment (start 109.347 91.313) (end 109.347 92.837) (width 0.25) (layer "B.Cu") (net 12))
 (segment (start 109.347 92.837) (end 111.526 95.016) (width 0.25) (layer "B.Cu") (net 12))
 (segment (start 108.077 90.043) (end 109.347 91.313) (width 0.25) (layer "B.Cu") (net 12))
 (segment (start 111.526 95.016) (end 114.413 95.016) (width 0.25) (layer "B.Cu") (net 12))
 (segment (start 105.585 92.61) (end 108.05 92.61) (width 0.25) (layer "F.Cu") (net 13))
 (segment (start 108.05 92.61) (end 108.077 92.583) (width 0.25) (layer "F.Cu") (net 13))
 (via (at 108.077 92.583) (size 0.43) (drill 0.2) (layers "F.Cu" "B.Cu") (free) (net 13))
 (segment (start 111.01 95.516) (end 114.413 95.516) (width 0.25) (layer "B.Cu") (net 13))
 (segment (start 108.077 92.583) (end 111.01 95.516) (width 0.25) (layer "B.Cu") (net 13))
 (segment (start 105.585 97.69) (end 108.05 97.69) (width 0.25) (layer "F.Cu") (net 14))
 (segment (start 108.05 97.69) (end 108.077 97.663) (width 0.25) (layer "F.Cu") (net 14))
 (via (at 108.077 97.663) (size 0.43) (drill 0.2) (layers "F.Cu" "B.Cu") (free) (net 14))
 (segment (start 109.724 96.016) (end 114.413 96.016) (width 0.25) (layer "B.Cu") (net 14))
 (segment (start 108.077 97.663) (end 109.724 96.016) (width 0.25) (layer "B.Cu") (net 14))
 (segment (start 105.585 100.23) (end 108.05 100.23) (width 0.25) (layer "F.Cu") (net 15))
 (segment (start 108.05 100.23) (end 108.077 100.203) (width 0.25) (layer "F.Cu") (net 15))
 (via (at 108.077 100.203) (size 0.43) (drill 0.2) (layers "F.Cu" "B.Cu") (free) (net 15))
 (segment (start 111.383 96.516) (end 114.413 96.516) (width 0.25) (layer "B.Cu") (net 15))
 (segment (start 109.093 99.187) (end 109.093 98.806) (width 0.25) (layer "B.Cu") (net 15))
 (segment (start 109.093 98.806) (end 111.383 96.516) (width 0.25) (layer "B.Cu") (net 15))
 (segment (start 108.077 100.203) (end 109.093 99.187) (width 0.25) (layer "B.Cu") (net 15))
 (segment (start 105.585 102.77) (end 108.05 102.77) (width 0.25) (layer "F.Cu") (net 16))
 (segment (start 108.05 102.77) (end 108.077 102.743) (width 0.25) (layer "F.Cu") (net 16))
 (via (at 108.077 102.743) (size 0.43) (drill 0.2) (layers "F.Cu" "B.Cu") (free) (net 16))
 (segment (start 108.077 102.743) (end 109.728 101.092) (width 0.25) (layer "B.Cu") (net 16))
 (segment (start 109.728 99.06) (end 111.772 97.016) (width 0.25) (layer "B.Cu") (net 16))
 (segment (start 111.772 97.016) (end 114.413 97.016) (width 0.25) (layer "B.Cu") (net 16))
 (segment (start 109.728 101.092) (end 109.728 99.06) (width 0.25) (layer "B.Cu") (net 16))
 (segment (start 105.585 105.31) (end 108.05 105.31) (width 0.25) (layer "F.Cu") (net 17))
 (segment (start 108.05 105.31) (end 108.077 105.283) (width 0.25) (layer "F.Cu") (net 17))
 (via (at 108.077 105.283) (size 0.43) (drill 0.2) (layers "F.Cu" "B.Cu") (free) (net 17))
 (segment (start 110.363 102.997) (end 110.363 99.314) (width 0.25) (layer "B.Cu") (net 17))
 (segment (start 112.161 97.516) (end 114.413 97.516) (width 0.25) (layer "B.Cu") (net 17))
 (segment (start 110.363 99.314) (end 112.161 97.516) (width 0.25) (layer "B.Cu") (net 17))
 (segment (start 108.077 105.283) (end 110.363 102.997) (width 0.25) (layer "B.Cu") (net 17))
 (segment (start 108.05 110.39) (end 108.077 110.363) (width 0.25) (layer "F.Cu") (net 18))
 (segment (start 105.585 110.39) (end 108.05 110.39) (width 0.25) (layer "F.Cu") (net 18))
 (via (at 108.077 110.363) (size 0.43) (drill 0.2) (layers "F.Cu" "B.Cu") (free) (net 18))
 (segment (start 110.998 99.568) (end 112.55 98.016) (width 0.25) (layer "B.Cu") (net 18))
 (segment (start 108.077 110.363) (end 110.998 107.442) (width 0.25) (layer "B.Cu") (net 18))
 (segment (start 112.55 98.016) (end 114.413 98.016) (width 0.25) (layer "B.Cu") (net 18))
 (segment (start 110.998 107.442) (end 110.998 99.568) (width 0.25) (layer "B.Cu") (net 18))
 (segment (start 107.923 112.93) (end 107.95 112.903) (width 0.25) (layer "F.Cu") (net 19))
 (segment (start 105.585 112.93) (end 107.923 112.93) (width 0.25) (layer "F.Cu") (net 19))
 (via (at 107.95 112.903) (size 0.43) (drill 0.2) (layers "F.Cu" "B.Cu") (free) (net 19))
 (segment (start 111.633 99.822) (end 112.939 98.516) (width 0.25) (layer "B.Cu") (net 19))
 (segment (start 112.939 98.516) (end 114.413 98.516) (width 0.25) (layer "B.Cu") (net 19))
 (segment (start 107.95 112.903) (end 111.633 109.22) (width 0.25) (layer "B.Cu") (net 19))
 (segment (start 111.633 109.22) (end 111.633 99.822) (width 0.25) (layer "B.Cu") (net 19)))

